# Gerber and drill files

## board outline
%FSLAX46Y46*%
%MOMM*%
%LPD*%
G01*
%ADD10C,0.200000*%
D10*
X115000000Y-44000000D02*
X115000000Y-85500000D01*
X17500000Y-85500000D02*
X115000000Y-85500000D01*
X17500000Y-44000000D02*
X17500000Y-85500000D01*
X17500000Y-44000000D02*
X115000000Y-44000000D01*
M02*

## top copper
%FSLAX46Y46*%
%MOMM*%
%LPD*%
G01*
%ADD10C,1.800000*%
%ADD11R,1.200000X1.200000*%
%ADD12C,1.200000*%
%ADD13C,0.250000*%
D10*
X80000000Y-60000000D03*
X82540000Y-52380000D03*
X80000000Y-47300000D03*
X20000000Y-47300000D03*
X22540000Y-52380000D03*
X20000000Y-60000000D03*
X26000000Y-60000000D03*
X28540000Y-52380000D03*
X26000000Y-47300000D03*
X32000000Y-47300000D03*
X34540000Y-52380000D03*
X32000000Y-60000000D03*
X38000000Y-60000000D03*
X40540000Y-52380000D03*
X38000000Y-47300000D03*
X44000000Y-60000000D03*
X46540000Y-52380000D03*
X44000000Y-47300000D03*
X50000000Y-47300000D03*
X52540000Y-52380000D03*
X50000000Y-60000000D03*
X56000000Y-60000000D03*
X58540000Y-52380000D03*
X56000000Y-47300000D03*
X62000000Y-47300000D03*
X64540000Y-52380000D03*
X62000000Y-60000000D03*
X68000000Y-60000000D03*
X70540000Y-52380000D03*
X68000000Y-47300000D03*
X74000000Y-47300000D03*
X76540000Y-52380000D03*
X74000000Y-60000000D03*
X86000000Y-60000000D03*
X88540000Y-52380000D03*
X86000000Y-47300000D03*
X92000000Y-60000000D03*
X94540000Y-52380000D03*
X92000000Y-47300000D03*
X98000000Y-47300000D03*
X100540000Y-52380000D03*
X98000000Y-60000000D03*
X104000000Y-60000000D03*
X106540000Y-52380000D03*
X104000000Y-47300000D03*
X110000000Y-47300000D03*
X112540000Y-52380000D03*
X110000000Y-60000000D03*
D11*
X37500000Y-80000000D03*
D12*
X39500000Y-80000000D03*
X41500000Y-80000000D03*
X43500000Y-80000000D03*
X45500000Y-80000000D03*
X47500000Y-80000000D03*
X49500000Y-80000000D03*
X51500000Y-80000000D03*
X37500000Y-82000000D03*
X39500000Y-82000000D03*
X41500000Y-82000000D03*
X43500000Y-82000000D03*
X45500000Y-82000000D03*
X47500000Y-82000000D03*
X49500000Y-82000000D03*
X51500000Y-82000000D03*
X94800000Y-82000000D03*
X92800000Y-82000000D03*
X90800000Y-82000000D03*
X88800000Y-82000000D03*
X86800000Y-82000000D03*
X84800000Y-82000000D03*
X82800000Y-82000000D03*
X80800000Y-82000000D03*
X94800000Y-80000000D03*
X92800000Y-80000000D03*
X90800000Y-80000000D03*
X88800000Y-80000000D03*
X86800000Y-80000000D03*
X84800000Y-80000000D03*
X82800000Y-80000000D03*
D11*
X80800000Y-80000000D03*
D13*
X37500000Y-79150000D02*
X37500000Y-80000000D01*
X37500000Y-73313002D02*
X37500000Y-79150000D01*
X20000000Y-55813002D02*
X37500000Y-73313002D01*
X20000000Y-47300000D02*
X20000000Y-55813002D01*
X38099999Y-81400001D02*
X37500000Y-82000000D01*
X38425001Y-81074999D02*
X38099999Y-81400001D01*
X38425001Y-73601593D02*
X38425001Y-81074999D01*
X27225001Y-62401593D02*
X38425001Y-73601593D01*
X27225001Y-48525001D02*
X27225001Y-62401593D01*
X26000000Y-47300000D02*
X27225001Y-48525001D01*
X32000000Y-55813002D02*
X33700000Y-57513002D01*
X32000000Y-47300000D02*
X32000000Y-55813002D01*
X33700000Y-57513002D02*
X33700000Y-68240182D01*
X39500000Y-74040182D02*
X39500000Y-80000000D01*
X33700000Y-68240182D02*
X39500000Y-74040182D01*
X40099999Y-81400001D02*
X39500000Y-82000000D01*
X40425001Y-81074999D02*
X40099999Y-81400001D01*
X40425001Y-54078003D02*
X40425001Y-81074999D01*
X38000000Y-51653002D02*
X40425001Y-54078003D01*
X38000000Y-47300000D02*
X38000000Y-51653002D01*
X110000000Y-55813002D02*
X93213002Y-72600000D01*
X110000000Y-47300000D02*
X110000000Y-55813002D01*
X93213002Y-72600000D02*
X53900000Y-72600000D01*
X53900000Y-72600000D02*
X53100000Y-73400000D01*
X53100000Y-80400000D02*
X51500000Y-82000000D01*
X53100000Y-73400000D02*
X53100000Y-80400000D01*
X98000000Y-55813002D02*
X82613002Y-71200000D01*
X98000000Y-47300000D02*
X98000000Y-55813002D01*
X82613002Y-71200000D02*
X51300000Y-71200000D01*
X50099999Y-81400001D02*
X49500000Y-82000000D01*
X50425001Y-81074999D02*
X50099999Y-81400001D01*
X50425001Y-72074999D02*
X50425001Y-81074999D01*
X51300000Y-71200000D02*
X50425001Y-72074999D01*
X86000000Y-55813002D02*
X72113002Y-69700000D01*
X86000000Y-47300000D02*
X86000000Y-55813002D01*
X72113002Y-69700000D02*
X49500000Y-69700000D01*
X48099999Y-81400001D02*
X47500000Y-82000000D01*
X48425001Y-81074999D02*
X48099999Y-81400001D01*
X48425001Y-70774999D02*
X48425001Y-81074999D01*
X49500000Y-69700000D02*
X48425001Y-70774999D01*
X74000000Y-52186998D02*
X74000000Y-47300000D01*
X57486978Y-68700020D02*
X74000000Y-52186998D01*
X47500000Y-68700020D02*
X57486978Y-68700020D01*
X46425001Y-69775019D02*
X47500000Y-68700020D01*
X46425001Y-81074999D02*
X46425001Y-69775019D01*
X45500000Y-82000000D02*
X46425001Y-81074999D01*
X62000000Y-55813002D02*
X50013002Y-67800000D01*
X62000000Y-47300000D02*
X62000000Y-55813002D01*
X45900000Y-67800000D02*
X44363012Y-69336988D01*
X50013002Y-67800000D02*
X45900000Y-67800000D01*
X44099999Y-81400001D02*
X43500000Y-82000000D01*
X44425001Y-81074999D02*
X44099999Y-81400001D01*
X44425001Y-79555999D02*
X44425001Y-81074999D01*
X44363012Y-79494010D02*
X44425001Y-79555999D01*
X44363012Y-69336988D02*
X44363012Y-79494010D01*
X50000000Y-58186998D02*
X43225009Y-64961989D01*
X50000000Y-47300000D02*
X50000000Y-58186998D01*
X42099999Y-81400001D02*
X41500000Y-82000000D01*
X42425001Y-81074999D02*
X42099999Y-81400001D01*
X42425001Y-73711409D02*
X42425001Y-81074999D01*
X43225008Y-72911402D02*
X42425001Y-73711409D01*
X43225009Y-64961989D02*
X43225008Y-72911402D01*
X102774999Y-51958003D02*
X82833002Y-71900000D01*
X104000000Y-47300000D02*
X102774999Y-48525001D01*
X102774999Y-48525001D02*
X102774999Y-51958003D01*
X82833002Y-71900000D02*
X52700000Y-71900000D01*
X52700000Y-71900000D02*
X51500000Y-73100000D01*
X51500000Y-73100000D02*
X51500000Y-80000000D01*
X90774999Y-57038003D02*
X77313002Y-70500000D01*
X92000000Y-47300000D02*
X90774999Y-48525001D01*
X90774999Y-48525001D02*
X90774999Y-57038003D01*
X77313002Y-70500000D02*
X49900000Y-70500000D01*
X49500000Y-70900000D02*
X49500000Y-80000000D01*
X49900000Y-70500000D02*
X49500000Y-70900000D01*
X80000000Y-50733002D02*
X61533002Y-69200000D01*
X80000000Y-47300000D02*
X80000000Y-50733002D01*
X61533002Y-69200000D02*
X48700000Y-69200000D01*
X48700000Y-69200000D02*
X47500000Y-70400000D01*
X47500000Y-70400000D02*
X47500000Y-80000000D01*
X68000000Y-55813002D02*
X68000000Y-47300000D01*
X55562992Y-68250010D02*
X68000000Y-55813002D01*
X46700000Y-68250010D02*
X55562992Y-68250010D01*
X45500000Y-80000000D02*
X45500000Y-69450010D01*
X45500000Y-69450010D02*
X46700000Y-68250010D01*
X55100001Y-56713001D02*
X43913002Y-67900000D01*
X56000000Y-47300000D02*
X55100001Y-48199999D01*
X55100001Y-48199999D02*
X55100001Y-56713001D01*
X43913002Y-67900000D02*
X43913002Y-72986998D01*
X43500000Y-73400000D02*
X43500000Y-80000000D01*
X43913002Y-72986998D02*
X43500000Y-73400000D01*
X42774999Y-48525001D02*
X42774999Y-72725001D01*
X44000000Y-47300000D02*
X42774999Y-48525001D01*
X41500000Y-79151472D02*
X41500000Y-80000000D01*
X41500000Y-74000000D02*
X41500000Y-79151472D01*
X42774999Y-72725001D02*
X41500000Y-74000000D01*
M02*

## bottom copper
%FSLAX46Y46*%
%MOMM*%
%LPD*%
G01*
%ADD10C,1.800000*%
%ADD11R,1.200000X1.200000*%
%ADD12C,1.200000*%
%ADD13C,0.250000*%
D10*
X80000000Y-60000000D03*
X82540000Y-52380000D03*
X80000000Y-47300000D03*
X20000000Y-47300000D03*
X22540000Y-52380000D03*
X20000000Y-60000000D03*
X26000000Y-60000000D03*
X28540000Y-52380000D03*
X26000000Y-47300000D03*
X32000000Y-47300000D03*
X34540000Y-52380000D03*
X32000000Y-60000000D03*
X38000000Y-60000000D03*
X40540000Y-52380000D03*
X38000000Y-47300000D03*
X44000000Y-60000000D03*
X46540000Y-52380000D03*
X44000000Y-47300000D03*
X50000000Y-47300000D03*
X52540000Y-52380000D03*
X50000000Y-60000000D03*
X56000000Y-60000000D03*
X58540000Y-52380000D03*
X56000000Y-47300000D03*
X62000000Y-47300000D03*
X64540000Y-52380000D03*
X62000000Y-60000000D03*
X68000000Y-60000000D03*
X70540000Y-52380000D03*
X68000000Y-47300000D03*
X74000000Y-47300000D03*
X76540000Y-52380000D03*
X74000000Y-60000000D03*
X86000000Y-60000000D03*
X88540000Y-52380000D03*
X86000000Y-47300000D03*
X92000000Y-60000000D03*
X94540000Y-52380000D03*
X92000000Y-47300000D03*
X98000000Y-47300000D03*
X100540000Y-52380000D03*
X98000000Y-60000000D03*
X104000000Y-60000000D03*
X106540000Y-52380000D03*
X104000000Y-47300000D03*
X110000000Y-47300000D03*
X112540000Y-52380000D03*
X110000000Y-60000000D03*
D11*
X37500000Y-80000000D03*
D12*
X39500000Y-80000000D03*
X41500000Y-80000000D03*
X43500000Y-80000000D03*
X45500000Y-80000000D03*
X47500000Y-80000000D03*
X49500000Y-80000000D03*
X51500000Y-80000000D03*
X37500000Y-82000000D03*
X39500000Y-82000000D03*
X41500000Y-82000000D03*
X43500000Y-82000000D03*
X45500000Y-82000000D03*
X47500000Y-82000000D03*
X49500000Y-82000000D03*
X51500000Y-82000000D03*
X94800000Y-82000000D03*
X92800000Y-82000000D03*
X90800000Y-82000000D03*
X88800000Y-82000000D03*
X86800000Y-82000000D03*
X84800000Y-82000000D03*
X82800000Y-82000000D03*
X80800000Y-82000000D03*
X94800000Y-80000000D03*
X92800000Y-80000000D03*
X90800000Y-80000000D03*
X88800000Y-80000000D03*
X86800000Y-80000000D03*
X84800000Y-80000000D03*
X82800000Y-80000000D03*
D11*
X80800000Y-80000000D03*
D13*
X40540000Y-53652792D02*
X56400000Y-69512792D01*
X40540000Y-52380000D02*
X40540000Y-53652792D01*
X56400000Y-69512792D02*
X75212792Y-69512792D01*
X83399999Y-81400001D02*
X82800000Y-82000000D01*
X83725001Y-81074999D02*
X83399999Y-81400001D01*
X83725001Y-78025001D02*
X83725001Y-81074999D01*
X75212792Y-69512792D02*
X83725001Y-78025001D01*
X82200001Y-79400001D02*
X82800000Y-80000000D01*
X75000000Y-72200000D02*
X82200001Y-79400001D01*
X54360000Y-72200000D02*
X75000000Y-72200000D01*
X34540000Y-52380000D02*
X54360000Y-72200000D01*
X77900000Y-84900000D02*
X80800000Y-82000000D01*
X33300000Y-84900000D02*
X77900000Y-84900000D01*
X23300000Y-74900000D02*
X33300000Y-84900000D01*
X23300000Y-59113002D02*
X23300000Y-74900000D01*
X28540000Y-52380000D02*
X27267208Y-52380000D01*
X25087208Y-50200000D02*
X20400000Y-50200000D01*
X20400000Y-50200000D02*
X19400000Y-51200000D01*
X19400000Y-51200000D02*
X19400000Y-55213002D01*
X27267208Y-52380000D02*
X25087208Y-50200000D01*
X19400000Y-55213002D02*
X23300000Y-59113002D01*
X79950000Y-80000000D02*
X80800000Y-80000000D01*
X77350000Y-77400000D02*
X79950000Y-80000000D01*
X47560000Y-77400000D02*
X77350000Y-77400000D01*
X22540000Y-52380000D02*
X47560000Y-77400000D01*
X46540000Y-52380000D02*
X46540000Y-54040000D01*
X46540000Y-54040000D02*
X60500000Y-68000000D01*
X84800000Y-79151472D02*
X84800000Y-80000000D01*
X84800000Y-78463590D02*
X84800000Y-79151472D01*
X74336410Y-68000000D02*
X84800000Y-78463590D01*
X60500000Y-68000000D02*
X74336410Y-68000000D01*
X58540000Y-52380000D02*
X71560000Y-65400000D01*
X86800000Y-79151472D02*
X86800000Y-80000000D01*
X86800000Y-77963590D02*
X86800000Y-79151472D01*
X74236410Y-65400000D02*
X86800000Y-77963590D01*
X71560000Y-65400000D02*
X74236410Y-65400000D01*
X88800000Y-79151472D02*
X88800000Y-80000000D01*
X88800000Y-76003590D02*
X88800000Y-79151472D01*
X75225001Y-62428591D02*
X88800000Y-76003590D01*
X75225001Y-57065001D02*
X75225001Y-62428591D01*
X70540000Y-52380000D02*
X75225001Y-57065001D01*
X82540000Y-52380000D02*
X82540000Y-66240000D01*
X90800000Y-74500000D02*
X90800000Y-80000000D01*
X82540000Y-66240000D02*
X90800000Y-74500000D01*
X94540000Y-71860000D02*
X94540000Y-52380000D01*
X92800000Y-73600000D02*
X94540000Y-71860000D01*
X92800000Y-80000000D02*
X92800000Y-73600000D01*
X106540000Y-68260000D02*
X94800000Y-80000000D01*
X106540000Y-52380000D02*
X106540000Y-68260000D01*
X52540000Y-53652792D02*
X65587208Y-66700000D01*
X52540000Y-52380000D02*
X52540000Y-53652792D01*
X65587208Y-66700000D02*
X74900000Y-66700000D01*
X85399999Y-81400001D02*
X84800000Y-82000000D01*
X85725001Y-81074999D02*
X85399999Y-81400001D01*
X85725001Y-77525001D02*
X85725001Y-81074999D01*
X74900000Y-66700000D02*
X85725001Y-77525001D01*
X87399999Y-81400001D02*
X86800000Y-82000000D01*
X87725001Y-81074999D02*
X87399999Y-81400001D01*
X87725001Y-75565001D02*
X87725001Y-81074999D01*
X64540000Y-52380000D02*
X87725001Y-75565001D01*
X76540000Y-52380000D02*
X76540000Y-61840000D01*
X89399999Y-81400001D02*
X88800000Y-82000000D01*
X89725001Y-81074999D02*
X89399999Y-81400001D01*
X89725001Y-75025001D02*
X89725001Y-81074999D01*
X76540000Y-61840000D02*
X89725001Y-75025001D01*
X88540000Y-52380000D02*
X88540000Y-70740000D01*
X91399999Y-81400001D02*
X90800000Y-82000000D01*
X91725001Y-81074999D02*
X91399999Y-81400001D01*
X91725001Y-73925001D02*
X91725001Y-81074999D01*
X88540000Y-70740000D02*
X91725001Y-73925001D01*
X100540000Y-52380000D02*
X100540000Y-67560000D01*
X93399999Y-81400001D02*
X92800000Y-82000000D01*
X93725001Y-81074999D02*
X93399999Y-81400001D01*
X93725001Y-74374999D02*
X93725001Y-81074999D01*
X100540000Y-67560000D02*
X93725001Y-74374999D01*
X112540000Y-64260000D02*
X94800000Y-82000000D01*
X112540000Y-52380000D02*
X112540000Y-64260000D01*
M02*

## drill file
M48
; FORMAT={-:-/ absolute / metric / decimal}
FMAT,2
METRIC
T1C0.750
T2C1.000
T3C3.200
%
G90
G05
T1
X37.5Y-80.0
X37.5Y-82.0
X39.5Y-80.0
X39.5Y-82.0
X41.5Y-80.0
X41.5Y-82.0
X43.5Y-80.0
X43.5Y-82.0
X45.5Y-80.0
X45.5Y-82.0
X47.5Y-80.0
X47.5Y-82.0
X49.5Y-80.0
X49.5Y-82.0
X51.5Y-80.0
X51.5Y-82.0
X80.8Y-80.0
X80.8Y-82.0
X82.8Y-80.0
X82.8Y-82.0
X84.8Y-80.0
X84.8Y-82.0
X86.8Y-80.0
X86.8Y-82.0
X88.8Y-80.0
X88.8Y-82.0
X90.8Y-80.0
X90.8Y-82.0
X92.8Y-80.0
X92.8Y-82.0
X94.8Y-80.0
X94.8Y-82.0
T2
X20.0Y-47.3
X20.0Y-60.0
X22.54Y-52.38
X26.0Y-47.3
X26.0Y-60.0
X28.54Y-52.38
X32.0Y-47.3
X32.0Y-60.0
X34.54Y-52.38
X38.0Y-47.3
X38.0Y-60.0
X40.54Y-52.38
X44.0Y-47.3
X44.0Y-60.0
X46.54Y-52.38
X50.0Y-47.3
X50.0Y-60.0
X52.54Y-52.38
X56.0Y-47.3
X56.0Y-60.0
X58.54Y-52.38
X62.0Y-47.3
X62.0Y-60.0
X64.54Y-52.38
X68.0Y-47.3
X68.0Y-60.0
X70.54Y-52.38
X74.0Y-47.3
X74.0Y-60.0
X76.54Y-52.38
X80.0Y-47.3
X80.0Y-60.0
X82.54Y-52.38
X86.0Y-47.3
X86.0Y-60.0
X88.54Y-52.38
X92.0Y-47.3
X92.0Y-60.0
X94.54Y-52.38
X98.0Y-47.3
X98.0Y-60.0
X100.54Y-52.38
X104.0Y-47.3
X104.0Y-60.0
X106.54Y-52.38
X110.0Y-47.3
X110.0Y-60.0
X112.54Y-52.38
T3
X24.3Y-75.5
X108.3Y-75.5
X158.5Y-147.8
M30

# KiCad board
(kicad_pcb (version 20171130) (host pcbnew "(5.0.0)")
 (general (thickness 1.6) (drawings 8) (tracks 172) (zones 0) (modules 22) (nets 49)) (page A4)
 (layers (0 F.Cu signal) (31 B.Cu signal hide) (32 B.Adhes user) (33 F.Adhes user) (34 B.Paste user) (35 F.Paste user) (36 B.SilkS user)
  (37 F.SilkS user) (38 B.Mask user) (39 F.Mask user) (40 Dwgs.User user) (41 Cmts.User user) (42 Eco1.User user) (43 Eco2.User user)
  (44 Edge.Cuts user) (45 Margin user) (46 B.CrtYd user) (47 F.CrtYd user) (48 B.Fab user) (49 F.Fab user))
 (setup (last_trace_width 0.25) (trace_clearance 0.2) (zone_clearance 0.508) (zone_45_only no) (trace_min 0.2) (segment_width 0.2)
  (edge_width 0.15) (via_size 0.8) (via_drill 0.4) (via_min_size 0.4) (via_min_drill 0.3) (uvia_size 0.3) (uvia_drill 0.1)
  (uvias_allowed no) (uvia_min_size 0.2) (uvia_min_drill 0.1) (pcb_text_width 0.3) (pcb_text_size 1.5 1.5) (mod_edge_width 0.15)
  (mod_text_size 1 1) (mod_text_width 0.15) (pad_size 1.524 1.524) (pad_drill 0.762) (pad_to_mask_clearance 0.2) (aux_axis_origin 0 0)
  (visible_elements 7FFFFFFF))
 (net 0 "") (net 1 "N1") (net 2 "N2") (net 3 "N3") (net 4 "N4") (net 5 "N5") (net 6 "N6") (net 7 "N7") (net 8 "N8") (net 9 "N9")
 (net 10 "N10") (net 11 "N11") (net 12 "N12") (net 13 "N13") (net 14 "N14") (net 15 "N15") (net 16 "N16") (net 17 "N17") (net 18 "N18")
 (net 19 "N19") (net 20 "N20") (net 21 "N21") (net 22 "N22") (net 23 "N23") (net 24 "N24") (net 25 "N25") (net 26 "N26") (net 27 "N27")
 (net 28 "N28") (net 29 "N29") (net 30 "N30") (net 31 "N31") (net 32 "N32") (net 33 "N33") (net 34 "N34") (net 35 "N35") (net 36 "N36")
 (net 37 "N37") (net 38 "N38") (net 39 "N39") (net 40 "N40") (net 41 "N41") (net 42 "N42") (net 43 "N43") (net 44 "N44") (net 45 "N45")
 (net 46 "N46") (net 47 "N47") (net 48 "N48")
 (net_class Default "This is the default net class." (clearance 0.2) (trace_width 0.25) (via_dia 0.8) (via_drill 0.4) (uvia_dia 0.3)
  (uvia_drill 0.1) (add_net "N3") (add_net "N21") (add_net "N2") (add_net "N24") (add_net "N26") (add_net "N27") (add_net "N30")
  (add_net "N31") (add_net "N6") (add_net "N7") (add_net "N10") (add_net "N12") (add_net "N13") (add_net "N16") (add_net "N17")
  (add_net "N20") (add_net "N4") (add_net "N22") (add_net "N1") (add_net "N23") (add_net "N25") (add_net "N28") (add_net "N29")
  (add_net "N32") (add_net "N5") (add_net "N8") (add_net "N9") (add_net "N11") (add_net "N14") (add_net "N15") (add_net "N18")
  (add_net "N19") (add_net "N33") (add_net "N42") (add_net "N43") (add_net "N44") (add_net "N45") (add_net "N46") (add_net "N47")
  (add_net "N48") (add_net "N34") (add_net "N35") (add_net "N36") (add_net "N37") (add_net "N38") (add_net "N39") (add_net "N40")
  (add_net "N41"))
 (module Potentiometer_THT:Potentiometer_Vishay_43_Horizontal (layer F.Cu) (at 80 60 270)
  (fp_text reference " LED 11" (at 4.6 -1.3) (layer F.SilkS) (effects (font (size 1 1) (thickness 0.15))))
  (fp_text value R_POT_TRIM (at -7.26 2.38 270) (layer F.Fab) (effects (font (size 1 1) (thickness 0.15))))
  (pad 1 thru_hole circle (at 0 0 270) (size 1.8 1.8) (drill 1) (layers *.Cu *.Mask))
  (pad 2 thru_hole circle (at -7.62 -2.54 270) (size 1.8 1.8) (drill 1) (layers *.Cu *.Mask) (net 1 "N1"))
  (pad 3 thru_hole circle (at -12.7 0 270) (size 1.8 1.8) (drill 1) (layers *.Cu *.Mask) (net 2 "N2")))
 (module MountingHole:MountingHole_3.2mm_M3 (layer F.Cu) (at 108.3 75.5)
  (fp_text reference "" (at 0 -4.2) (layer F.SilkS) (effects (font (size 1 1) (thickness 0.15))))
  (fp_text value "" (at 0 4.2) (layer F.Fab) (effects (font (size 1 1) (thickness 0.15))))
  (pad 1 np_thru_hole circle (at 0 0) (size 3.2 3.2) (drill 3.2) (layers *.Cu *.Mask)))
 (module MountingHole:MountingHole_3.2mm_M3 (layer F.Cu) (at 24.3 75.5)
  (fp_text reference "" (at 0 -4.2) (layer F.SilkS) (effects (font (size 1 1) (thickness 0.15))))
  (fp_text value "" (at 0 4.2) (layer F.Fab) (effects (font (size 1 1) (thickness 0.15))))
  (pad 1 np_thru_hole circle (at 0 0) (size 3.2 3.2) (drill 3.2) (layers *.Cu *.Mask)))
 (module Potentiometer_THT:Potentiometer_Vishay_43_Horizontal (layer F.Cu) (at 20 60 270)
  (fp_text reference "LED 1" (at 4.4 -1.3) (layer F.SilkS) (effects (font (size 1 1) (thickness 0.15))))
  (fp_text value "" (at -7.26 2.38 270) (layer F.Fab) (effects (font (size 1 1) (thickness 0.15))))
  (pad 3 thru_hole circle (at -12.7 0 270) (size 1.8 1.8) (drill 1) (layers *.Cu *.Mask) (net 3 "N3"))
  (pad 2 thru_hole circle (at -7.62 -2.54 270) (size 1.8 1.8) (drill 1) (layers *.Cu *.Mask) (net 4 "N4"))
  (pad 1 thru_hole circle (at 0 0 270) (size 1.8 1.8) (drill 1) (layers *.Cu *.Mask)))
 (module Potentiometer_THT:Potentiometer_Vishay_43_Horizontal (layer F.Cu) (at 26 60 270)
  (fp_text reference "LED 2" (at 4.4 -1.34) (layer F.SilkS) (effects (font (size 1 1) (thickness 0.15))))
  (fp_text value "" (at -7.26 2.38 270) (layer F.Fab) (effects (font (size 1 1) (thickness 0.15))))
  (pad 1 thru_hole circle (at 0 0 270) (size 1.8 1.8) (drill 1) (layers *.Cu *.Mask))
  (pad 2 thru_hole circle (at -7.62 -2.54 270) (size 1.8 1.8) (drill 1) (layers *.Cu *.Mask) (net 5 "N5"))
  (pad 3 thru_hole circle (at -12.7 0 270) (size 1.8 1.8) (drill 1) (layers *.Cu *.Mask) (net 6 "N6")))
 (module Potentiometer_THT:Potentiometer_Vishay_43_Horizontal (layer F.Cu) (at 32 60 270)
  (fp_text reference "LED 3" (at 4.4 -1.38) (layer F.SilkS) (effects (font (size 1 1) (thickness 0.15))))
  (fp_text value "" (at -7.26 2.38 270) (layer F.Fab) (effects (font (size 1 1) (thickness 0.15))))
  (pad 3 thru_hole circle (at -12.7 0 270) (size 1.8 1.8) (drill 1) (layers *.Cu *.Mask) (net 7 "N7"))
  (pad 2 thru_hole circle (at -7.62 -2.54 270) (size 1.8 1.8) (drill 1) (layers *.Cu *.Mask) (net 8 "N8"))
  (pad 1 thru_hole circle (at 0 0 270) (size 1.8 1.8) (drill 1) (layers *.Cu *.Mask)))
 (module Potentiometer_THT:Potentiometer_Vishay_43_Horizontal (layer F.Cu) (at 38 60 270)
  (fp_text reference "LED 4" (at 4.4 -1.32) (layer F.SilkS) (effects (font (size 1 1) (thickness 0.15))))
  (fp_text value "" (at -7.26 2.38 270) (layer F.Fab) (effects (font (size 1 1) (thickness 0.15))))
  (pad 1 thru_hole circle (at 0 0 270) (size 1.8 1.8) (drill 1) (layers *.Cu *.Mask))
  (pad 2 thru_hole circle (at -7.62 -2.54 270) (size 1.8 1.8) (drill 1) (layers *.Cu *.Mask) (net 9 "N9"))
  (pad 3 thru_hole circle (at -12.7 0 270) (size 1.8 1.8) (drill 1) (layers *.Cu *.Mask) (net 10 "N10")))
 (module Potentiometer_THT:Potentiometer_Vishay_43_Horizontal (layer F.Cu) (at 44 60 270)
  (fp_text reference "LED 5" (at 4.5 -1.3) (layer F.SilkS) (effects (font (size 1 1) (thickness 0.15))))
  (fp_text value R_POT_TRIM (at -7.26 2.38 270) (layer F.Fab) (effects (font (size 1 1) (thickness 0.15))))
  (pad 1 thru_hole circle (at 0 0 270) (size 1.8 1.8) (drill 1) (layers *.Cu *.Mask))
  (pad 2 thru_hole circle (at -7.62 -2.54 270) (size 1.8 1.8) (drill 1) (layers *.Cu *.Mask) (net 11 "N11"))
  (pad 3 thru_hole circle (at -12.7 0 270) (size 1.8 1.8) (drill 1) (layers *.Cu *.Mask) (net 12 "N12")))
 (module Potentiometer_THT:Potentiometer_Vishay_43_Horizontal (layer F.Cu) (at 50 60 270)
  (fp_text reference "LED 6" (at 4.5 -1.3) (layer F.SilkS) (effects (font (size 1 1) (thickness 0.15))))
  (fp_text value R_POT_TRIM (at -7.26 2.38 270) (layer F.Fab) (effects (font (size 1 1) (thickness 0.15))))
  (pad 3 thru_hole circle (at -12.7 0 270) (size 1.8 1.8) (drill 1) (layers *.Cu *.Mask) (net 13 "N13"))
  (pad 2 thru_hole circle (at -7.62 -2.54 270) (size 1.8 1.8) (drill 1) (layers *.Cu *.Mask) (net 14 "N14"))
  (pad 1 thru_hole circle (at 0 0 270) (size 1.8 1.8) (drill 1) (layers *.Cu *.Mask)))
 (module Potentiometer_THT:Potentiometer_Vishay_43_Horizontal (layer F.Cu) (at 56 60 270)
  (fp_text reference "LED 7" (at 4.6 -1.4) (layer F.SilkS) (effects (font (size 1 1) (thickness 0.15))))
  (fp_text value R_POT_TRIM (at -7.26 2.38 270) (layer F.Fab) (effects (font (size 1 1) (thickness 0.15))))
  (pad 1 thru_hole circle (at 0 0 270) (size 1.8 1.8) (drill 1) (layers *.Cu *.Mask))
  (pad 2 thru_hole circle (at -7.62 -2.54 270) (size 1.8 1.8) (drill 1) (layers *.Cu *.Mask) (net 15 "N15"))
  (pad 3 thru_hole circle (at -12.7 0 270) (size 1.8 1.8) (drill 1) (layers *.Cu *.Mask) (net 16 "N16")))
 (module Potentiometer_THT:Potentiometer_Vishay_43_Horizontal (layer F.Cu) (at 62 60 270)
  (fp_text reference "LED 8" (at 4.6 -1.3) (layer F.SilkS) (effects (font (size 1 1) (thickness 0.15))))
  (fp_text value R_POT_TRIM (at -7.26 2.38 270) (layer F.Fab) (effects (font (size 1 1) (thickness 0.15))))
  (pad 3 thru_hole circle (at -12.7 0 270) (size 1.8 1.8) (drill 1) (layers *.Cu *.Mask) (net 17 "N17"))
  (pad 2 thru_hole circle (at -7.62 -2.54 270) (size 1.8 1.8) (drill 1) (layers *.Cu *.Mask) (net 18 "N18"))
  (pad 1 thru_hole circle (at 0 0 270) (size 1.8 1.8) (drill 1) (layers *.Cu *.Mask)))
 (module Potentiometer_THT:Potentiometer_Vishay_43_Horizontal (layer F.Cu) (at 68 60 270)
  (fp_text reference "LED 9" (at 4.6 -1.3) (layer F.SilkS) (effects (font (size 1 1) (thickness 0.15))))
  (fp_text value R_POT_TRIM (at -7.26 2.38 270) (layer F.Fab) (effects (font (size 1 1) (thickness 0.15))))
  (pad 1 thru_hole circle (at 0 0 270) (size 1.8 1.8) (drill 1) (layers *.Cu *.Mask))
  (pad 2 thru_hole circle (at -7.62 -2.54 270) (size 1.8 1.8) (drill 1) (layers *.Cu *.Mask) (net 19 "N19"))
  (pad 3 thru_hole circle (at -12.7 0 270) (size 1.8 1.8) (drill 1) (layers *.Cu *.Mask) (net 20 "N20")))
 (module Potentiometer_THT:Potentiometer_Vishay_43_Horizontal (layer F.Cu) (at 74 60 270)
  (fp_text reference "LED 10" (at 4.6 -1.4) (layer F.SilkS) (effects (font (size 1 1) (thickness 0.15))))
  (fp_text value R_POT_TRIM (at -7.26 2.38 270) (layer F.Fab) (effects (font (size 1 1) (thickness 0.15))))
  (pad 3 thru_hole circle (at -12.7 0 270) (size 1.8 1.8) (drill 1) (layers *.Cu *.Mask) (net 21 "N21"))
  (pad 2 thru_hole circle (at -7.62 -2.54 270) (size 1.8 1.8) (drill 1) (layers *.Cu *.Mask) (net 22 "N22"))
  (pad 1 thru_hole circle (at 0 0 270) (size 1.8 1.8) (drill 1) (layers *.Cu *.Mask)))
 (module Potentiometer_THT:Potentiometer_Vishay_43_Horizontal (layer F.Cu) (at 86 60 270)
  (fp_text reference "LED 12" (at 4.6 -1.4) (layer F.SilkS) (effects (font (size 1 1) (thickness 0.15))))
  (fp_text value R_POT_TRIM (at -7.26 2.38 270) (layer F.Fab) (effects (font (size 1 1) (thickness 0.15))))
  (pad 1 thru_hole circle (at 0 0 270) (size 1.8 1.8) (drill 1) (layers *.Cu *.Mask))
  (pad 2 thru_hole circle (at -7.62 -2.54 270) (size 1.8 1.8) (drill 1) (layers *.Cu *.Mask) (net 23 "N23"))
  (pad 3 thru_hole circle (at -12.7 0 270) (size 1.8 1.8) (drill 1) (layers *.Cu *.Mask) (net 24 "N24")))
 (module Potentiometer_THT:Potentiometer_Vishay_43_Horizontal (layer F.Cu) (at 92 60 270)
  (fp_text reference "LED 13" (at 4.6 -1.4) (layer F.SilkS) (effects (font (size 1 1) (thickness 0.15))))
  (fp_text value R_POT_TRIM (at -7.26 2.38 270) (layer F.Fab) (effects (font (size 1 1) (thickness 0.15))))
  (pad 1 thru_hole circle (at 0 0 270) (size 1.8 1.8) (drill 1) (layers *.Cu *.Mask))
  (pad 2 thru_hole circle (at -7.62 -2.54 270) (size 1.8 1.8) (drill 1) (layers *.Cu *.Mask) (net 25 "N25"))
  (pad 3 thru_hole circle (at -12.7 0 270) (size 1.8 1.8) (drill 1) (layers *.Cu *.Mask) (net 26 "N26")))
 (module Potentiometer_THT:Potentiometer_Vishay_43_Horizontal (layer F.Cu) (at 98 60 270)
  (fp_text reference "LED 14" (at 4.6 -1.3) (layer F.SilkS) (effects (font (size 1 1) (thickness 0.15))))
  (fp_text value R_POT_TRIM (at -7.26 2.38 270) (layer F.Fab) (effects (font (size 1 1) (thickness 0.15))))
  (pad 3 thru_hole circle (at -12.7 0 270) (size 1.8 1.8) (drill 1) (layers *.Cu *.Mask) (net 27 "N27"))
  (pad 2 thru_hole circle (at -7.62 -2.54 270) (size 1.8 1.8) (drill 1) (layers *.Cu *.Mask) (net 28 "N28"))
  (pad 1 thru_hole circle (at 0 0 270) (size 1.8 1.8) (drill 1) (layers *.Cu *.Mask)))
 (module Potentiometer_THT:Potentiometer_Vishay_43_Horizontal (layer F.Cu) (at 104 60 270)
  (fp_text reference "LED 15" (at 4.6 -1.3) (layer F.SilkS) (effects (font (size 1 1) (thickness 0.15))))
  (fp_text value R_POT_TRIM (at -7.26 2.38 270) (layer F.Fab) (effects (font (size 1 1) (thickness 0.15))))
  (pad 1 thru_hole circle (at 0 0 270) (size 1.8 1.8) (drill 1) (layers *.Cu *.Mask))
  (pad 2 thru_hole circle (at -7.62 -2.54 270) (size 1.8 1.8) (drill 1) (layers *.Cu *.Mask) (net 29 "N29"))
  (pad 3 thru_hole circle (at -12.7 0 270) (size 1.8 1.8) (drill 1) (layers *.Cu *.Mask) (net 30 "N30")))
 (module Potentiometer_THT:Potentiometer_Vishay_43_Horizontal (layer F.Cu) (at 110 60 270)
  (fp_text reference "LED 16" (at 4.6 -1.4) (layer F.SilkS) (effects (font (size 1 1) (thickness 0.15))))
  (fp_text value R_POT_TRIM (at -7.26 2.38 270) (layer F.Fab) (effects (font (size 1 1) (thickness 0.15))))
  (pad 3 thru_hole circle (at -12.7 0 270) (size 1.8 1.8) (drill 1) (layers *.Cu *.Mask) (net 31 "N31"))
  (pad 2 thru_hole circle (at -7.62 -2.54 270) (size 1.8 1.8) (drill 1) (layers *.Cu *.Mask) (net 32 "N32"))
  (pad 1 thru_hole circle (at 0 0 270) (size 1.8 1.8) (drill 1) (layers *.Cu *.Mask)))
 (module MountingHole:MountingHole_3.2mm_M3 (layer F.Cu) (at 158.5 147.8)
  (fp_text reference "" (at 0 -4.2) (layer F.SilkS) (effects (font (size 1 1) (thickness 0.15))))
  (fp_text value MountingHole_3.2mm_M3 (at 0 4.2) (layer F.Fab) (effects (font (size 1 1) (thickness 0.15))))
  (pad 1 np_thru_hole circle (at 0 0) (size 3.2 3.2) (drill 3.2) (layers *.Cu *.Mask)))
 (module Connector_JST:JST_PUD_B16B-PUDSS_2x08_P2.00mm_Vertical (layer F.Cu) (at 37.5 80)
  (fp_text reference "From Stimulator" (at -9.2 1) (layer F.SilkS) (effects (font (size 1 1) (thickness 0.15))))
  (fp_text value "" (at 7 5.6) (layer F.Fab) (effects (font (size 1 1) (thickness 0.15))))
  (pad 1 thru_hole rect (at 0 0) (size 1.2 1.2) (drill 0.75) (layers *.Cu *.Mask) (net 3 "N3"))
  (pad 3 thru_hole circle (at 2 0) (size 1.2 1.2) (drill 0.75) (layers *.Cu *.Mask) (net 7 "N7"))
  (pad 5 thru_hole circle (at 4 0) (size 1.2 1.2) (drill 0.75) (layers *.Cu *.Mask) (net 12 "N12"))
  (pad 7 thru_hole circle (at 6 0) (size 1.2 1.2) (drill 0.75) (layers *.Cu *.Mask) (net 16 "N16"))
  (pad 9 thru_hole circle (at 8 0) (size 1.2 1.2) (drill 0.75) (layers *.Cu *.Mask) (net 20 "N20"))
  (pad 11 thru_hole circle (at 10 0) (size 1.2 1.2) (drill 0.75) (layers *.Cu *.Mask) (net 2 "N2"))
  (pad 13 thru_hole circle (at 12 0) (size 1.2 1.2) (drill 0.75) (layers *.Cu *.Mask) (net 26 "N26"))
  (pad 15 thru_hole circle (at 14 0) (size 1.2 1.2) (drill 0.75) (layers *.Cu *.Mask) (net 30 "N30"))
  (pad 2 thru_hole circle (at 0 2) (size 1.2 1.2) (drill 0.75) (layers *.Cu *.Mask) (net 6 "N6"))
  (pad 4 thru_hole circle (at 2 2) (size 1.2 1.2) (drill 0.75) (layers *.Cu *.Mask) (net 10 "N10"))
  (pad 6 thru_hole circle (at 4 2) (size 1.2 1.2) (drill 0.75) (layers *.Cu *.Mask) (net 13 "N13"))
  (pad 8 thru_hole circle (at 6 2) (size 1.2 1.2) (drill 0.75) (layers *.Cu *.Mask) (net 17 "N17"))
  (pad 10 thru_hole circle (at 8 2) (size 1.2 1.2) (drill 0.75) (layers *.Cu *.Mask) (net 21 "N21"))
  (pad 12 thru_hole circle (at 10 2) (size 1.2 1.2) (drill 0.75) (layers *.Cu *.Mask) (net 24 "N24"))
  (pad 14 thru_hole circle (at 12 2) (size 1.2 1.2) (drill 0.75) (layers *.Cu *.Mask) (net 27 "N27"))
  (pad 16 thru_hole circle (at 14 2) (size 1.2 1.2) (drill 0.75) (layers *.Cu *.Mask) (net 31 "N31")))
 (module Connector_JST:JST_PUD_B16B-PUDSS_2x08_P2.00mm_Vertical (layer F.Cu) (at 80.8 80)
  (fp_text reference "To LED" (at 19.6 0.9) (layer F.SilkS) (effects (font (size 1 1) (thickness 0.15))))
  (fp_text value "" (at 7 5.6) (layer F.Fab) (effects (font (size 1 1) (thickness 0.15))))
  (pad 16 thru_hole circle (at 14 2) (size 1.2 1.2) (drill 0.75) (layers *.Cu *.Mask) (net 32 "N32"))
  (pad 14 thru_hole circle (at 12 2) (size 1.2 1.2) (drill 0.75) (layers *.Cu *.Mask) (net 28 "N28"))
  (pad 12 thru_hole circle (at 10 2) (size 1.2 1.2) (drill 0.75) (layers *.Cu *.Mask) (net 23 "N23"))
  (pad 10 thru_hole circle (at 8 2) (size 1.2 1.2) (drill 0.75) (layers *.Cu *.Mask) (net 22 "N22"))
  (pad 8 thru_hole circle (at 6 2) (size 1.2 1.2) (drill 0.75) (layers *.Cu *.Mask) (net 18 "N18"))
  (pad 6 thru_hole circle (at 4 2) (size 1.2 1.2) (drill 0.75) (layers *.Cu *.Mask) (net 14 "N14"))
  (pad 4 thru_hole circle (at 2 2) (size 1.2 1.2) (drill 0.75) (layers *.Cu *.Mask) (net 9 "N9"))
  (pad 2 thru_hole circle (at 0 2) (size 1.2 1.2) (drill 0.75) (layers *.Cu *.Mask) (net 5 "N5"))
  (pad 15 thru_hole circle (at 14 0) (size 1.2 1.2) (drill 0.75) (layers *.Cu *.Mask) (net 29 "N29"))
  (pad 13 thru_hole circle (at 12 0) (size 1.2 1.2) (drill 0.75) (layers *.Cu *.Mask) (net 25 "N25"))
  (pad 11 thru_hole circle (at 10 0) (size 1.2 1.2) (drill 0.75) (layers *.Cu *.Mask) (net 1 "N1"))
  (pad 9 thru_hole circle (at 8 0) (size 1.2 1.2) (drill 0.75) (layers *.Cu *.Mask) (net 19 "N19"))
  (pad 7 thru_hole circle (at 6 0) (size 1.2 1.2) (drill 0.75) (layers *.Cu *.Mask) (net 15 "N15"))
  (pad 5 thru_hole circle (at 4 0) (size 1.2 1.2) (drill 0.75) (layers *.Cu *.Mask) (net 11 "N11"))
  (pad 3 thru_hole circle (at 2 0) (size 1.2 1.2) (drill 0.75) (layers *.Cu *.Mask) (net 8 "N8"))
  (pad 1 thru_hole rect (at 0 0) (size 1.2 1.2) (drill 0.75) (layers *.Cu *.Mask) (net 4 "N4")))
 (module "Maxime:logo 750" (layer F.Cu) (at 67.8 80.4)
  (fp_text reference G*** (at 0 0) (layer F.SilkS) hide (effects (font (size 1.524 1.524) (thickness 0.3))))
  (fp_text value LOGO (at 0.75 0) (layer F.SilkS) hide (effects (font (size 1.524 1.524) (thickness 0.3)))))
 (gr_line (start 115 44) (end 115 85.5) (layer Edge.Cuts) (width 0.2))
 (gr_line (start 17.5 85.5) (end 115 85.5) (layer Edge.Cuts) (width 0.2))
 (gr_line (start 17.5 44) (end 17.5 85.5) (layer Edge.Cuts) (width 0.2))
 (gr_line (start 17.5 44) (end 115 44) (layer Edge.Cuts) (width 0.2))
 (segment (start 37.5 79.15) (end 37.5 80) (width 0.25) (layer F.Cu) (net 3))
 (segment (start 37.5 73.313002) (end 37.5 79.15) (width 0.25) (layer F.Cu) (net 3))
 (segment (start 20 55.813002) (end 37.5 73.313002) (width 0.25) (layer F.Cu) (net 3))
 (segment (start 20 47.3) (end 20 55.813002) (width 0.25) (layer F.Cu) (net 3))
 (segment (start 38.099999 81.400001) (end 37.5 82) (width 0.25) (layer F.Cu) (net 6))
 (segment (start 38.425001 81.074999) (end 38.099999 81.400001) (width 0.25) (layer F.Cu) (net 6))
 (segment (start 38.425001 73.601593) (end 38.425001 81.074999) (width 0.25) (layer F.Cu) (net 6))
 (segment (start 27.225001 62.401593) (end 38.425001 73.601593) (width 0.25) (layer F.Cu) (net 6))
 (segment (start 27.225001 48.525001) (end 27.225001 62.401593) (width 0.25) (layer F.Cu) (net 6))
 (segment (start 26 47.3) (end 27.225001 48.525001) (width 0.25) (layer F.Cu) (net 6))
 (segment (start 32 55.813002) (end 33.7 57.513002) (width 0.25) (layer F.Cu) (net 7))
 (segment (start 32 47.3) (end 32 55.813002) (width 0.25) (layer F.Cu) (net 7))
 (segment (start 33.7 57.513002) (end 33.7 68.240182) (width 0.25) (layer F.Cu) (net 7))
 (segment (start 39.5 74.040182) (end 39.5 80) (width 0.25) (layer F.Cu) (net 7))
 (segment (start 33.7 68.240182) (end 39.5 74.040182) (width 0.25) (layer F.Cu) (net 7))
 (segment (start 40.099999 81.400001) (end 39.5 82) (width 0.25) (layer F.Cu) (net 10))
 (segment (start 40.425001 81.074999) (end 40.099999 81.400001) (width 0.25) (layer F.Cu) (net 10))
 (segment (start 40.425001 54.078003) (end 40.425001 81.074999) (width 0.25) (layer F.Cu) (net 10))
 (segment (start 38 51.653002) (end 40.425001 54.078003) (width 0.25) (layer F.Cu) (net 10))
 (segment (start 38 47.3) (end 38 51.653002) (width 0.25) (layer F.Cu) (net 10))
 (segment (start 40.54 53.652792) (end 56.4 69.512792) (width 0.25) (layer B.Cu) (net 9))
 (segment (start 40.54 52.38) (end 40.54 53.652792) (width 0.25) (layer B.Cu) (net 9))
 (segment (start 56.4 69.512792) (end 75.212792 69.512792) (width 0.25) (layer B.Cu) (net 9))
 (segment (start 83.399999 81.400001) (end 82.8 82) (width 0.25) (layer B.Cu) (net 9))
 (segment (start 83.725001 81.074999) (end 83.399999 81.400001) (width 0.25) (layer B.Cu) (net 9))
 (segment (start 83.725001 78.025001) (end 83.725001 81.074999) (width 0.25) (layer B.Cu) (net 9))
 (segment (start 75.212792 69.512792) (end 83.725001 78.025001) (width 0.25) (layer B.Cu) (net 9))
 (segment (start 82.200001 79.400001) (end 82.8 80) (width 0.25) (layer B.Cu) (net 8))
 (segment (start 75 72.2) (end 82.200001 79.400001) (width 0.25) (layer B.Cu) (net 8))
 (segment (start 54.36 72.2) (end 75 72.2) (width 0.25) (layer B.Cu) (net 8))
 (segment (start 34.54 52.38) (end 54.36 72.2) (width 0.25) (layer B.Cu) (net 8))
 (segment (start 77.9 84.9) (end 80.8 82) (width 0.25) (layer B.Cu) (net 5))
 (segment (start 33.3 84.9) (end 77.9 84.9) (width 0.25) (layer B.Cu) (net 5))
 (segment (start 23.3 74.9) (end 33.3 84.9) (width 0.25) (layer B.Cu) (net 5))
 (segment (start 23.3 59.113002) (end 23.3 74.9) (width 0.25) (layer B.Cu) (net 5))
 (segment (start 28.54 52.38) (end 27.267208 52.38) (width 0.25) (layer B.Cu) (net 5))
 (segment (start 25.087208 50.2) (end 20.4 50.2) (width 0.25) (layer B.Cu) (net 5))
 (segment (start 20.4 50.2) (end 19.4 51.2) (width 0.25) (layer B.Cu) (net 5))
 (segment (start 19.4 51.2) (end 19.4 55.213002) (width 0.25) (layer B.Cu) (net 5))
 (segment (start 27.267208 52.38) (end 25.087208 50.2) (width 0.25) (layer B.Cu) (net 5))
 (segment (start 19.4 55.213002) (end 23.3 59.113002) (width 0.25) (layer B.Cu) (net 5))
 (segment (start 79.95 80) (end 80.8 80) (width 0.25) (layer B.Cu) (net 4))
 (segment (start 77.35 77.4) (end 79.95 80) (width 0.25) (layer B.Cu) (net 4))
 (segment (start 47.56 77.4) (end 77.35 77.4) (width 0.25) (layer B.Cu) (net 4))
 (segment (start 22.54 52.38) (end 47.56 77.4) (width 0.25) (layer B.Cu) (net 4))
 (segment (start 110 55.813002) (end 93.213002 72.6) (width 0.25) (layer F.Cu) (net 31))
 (segment (start 110 47.3) (end 110 55.813002) (width 0.25) (layer F.Cu) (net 31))
 (segment (start 93.213002 72.6) (end 53.9 72.6) (width 0.25) (layer F.Cu) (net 31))
 (segment (start 53.9 72.6) (end 53.1 73.4) (width 0.25) (layer F.Cu) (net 31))
 (segment (start 53.1 80.4) (end 51.5 82) (width 0.25) (layer F.Cu) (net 31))
 (segment (start 53.1 73.4) (end 53.1 80.4) (width 0.25) (layer F.Cu) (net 31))
 (segment (start 98 55.813002) (end 82.613002 71.2) (width 0.25) (layer F.Cu) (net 27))
 (segment (start 98 47.3) (end 98 55.813002) (width 0.25) (layer F.Cu) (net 27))
 (segment (start 82.613002 71.2) (end 51.3 71.2) (width 0.25) (layer F.Cu) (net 27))
 (segment (start 50.099999 81.400001) (end 49.5 82) (width 0.25) (layer F.Cu) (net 27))
 (segment (start 50.425001 81.074999) (end 50.099999 81.400001) (width 0.25) (layer F.Cu) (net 27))
 (segment (start 50.425001 72.074999) (end 50.425001 81.074999) (width 0.25) (layer F.Cu) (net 27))
 (segment (start 51.3 71.2) (end 50.425001 72.074999) (width 0.25) (layer F.Cu) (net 27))
 (segment (start 86 55.813002) (end 72.113002 69.7) (width 0.25) (layer F.Cu) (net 24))
 (segment (start 86 47.3) (end 86 55.813002) (width 0.25) (layer F.Cu) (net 24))
 (segment (start 72.113002 69.7) (end 49.5 69.7) (width 0.25) (layer F.Cu) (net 24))
 (segment (start 48.099999 81.400001) (end 47.5 82) (width 0.25) (layer F.Cu) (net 24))
 (segment (start 48.425001 81.074999) (end 48.099999 81.400001) (width 0.25) (layer F.Cu) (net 24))
 (segment (start 48.425001 70.774999) (end 48.425001 81.074999) (width 0.25) (layer F.Cu) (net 24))
 (segment (start 49.5 69.7) (end 48.425001 70.774999) (width 0.25) (layer F.Cu) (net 24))
 (segment (start 74 52.186998) (end 74 47.3) (width 0.25) (layer F.Cu) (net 21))
 (segment (start 57.486978 68.70002) (end 74 52.186998) (width 0.25) (layer F.Cu) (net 21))
 (segment (start 47.5 68.70002) (end 57.486978 68.70002) (width 0.25) (layer F.Cu) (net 21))
 (segment (start 46.425001 69.775019) (end 47.5 68.70002) (width 0.25) (layer F.Cu) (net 21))
 (segment (start 46.425001 81.074999) (end 46.425001 69.775019) (width 0.25) (layer F.Cu) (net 21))
 (segment (start 45.5 82) (end 46.425001 81.074999) (width 0.25) (layer F.Cu) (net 21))
 (segment (start 62 55.813002) (end 50.013002 67.8) (width 0.25) (layer F.Cu) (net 17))
 (segment (start 62 47.3) (end 62 55.813002) (width 0.25) (layer F.Cu) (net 17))
 (segment (start 45.9 67.8) (end 44.363012 69.336988) (width 0.25) (layer F.Cu) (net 17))
 (segment (start 50.013002 67.8) (end 45.9 67.8) (width 0.25) (layer F.Cu) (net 17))
 (segment (start 44.099999 81.400001) (end 43.5 82) (width 0.25) (layer F.Cu) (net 17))
 (segment (start 44.425001 81.074999) (end 44.099999 81.400001) (width 0.25) (layer F.Cu) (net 17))
 (segment (start 44.425001 79.555999) (end 44.425001 81.074999) (width 0.25) (layer F.Cu) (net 17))
 (segment (start 44.363012 79.49401) (end 44.425001 79.555999) (width 0.25) (layer F.Cu) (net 17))
 (segment (start 44.363012 69.336988) (end 44.363012 79.49401) (width 0.25) (layer F.Cu) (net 17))
 (segment (start 50 58.186998) (end 43.225009 64.961989) (width 0.25) (layer F.Cu) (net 13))
 (segment (start 50 47.3) (end 50 58.186998) (width 0.25) (layer F.Cu) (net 13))
 (segment (start 42.099999 81.400001) (end 41.5 82) (width 0.25) (layer F.Cu) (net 13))
 (segment (start 42.425001 81.074999) (end 42.099999 81.400001) (width 0.25) (layer F.Cu) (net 13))
 (segment (start 42.425001 73.711409) (end 42.425001 81.074999) (width 0.25) (layer F.Cu) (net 13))
 (segment (start 43.225008 72.911402) (end 42.425001 73.711409) (width 0.25) (layer F.Cu) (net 13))
 (segment (start 43.225009 64.961989) (end 43.225008 72.911402) (width 0.25) (layer F.Cu) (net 13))
 (segment (start 102.774999 51.958003) (end 82.833002 71.9) (width 0.25) (layer F.Cu) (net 30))
 (segment (start 104 47.3) (end 102.774999 48.525001) (width 0.25) (layer F.Cu) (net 30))
 (segment (start 102.774999 48.525001) (end 102.774999 51.958003) (width 0.25) (layer F.Cu) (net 30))
 (segment (start 82.833002 71.9) (end 52.7 71.9) (width 0.25) (layer F.Cu) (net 30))
 (segment (start 52.7 71.9) (end 51.5 73.1) (width 0.25) (layer F.Cu) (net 30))
 (segment (start 51.5 73.1) (end 51.5 80) (width 0.25) (layer F.Cu) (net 30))
 (segment (start 90.774999 57.038003) (end 77.313002 70.5) (width 0.25) (layer F.Cu) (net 26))
 (segment (start 92 47.3) (end 90.774999 48.525001) (width 0.25) (layer F.Cu) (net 26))
 (segment (start 90.774999 48.525001) (end 90.774999 57.038003) (width 0.25) (layer F.Cu) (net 26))
 (segment (start 77.313002 70.5) (end 49.9 70.5) (width 0.25) (layer F.Cu) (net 26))
 (segment (start 49.5 70.9) (end 49.5 80) (width 0.25) (layer F.Cu) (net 26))
 (segment (start 49.9 70.5) (end 49.5 70.9) (width 0.25) (layer F.Cu) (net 26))
 (segment (start 80 50.733002) (end 61.533002 69.2) (width 0.25) (layer F.Cu) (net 2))
 (segment (start 80 47.3) (end 80 50.733002) (width 0.25) (layer F.Cu) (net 2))
 (segment (start 61.533002 69.2) (end 48.7 69.2) (width 0.25) (layer F.Cu) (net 2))
 (segment (start 48.7 69.2) (end 47.5 70.4) (width 0.25) (layer F.Cu) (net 2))
 (segment (start 47.5 70.4) (end 47.5 80) (width 0.25) (layer F.Cu) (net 2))
 (segment (start 68 55.813002) (end 68 47.3) (width 0.25) (layer F.Cu) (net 20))
 (segment (start 55.562992 68.25001) (end 68 55.813002) (width 0.25) (layer F.Cu) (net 20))
 (segment (start 46.7 68.25001) (end 55.562992 68.25001) (width 0.25) (layer F.Cu) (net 20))
 (segment (start 45.5 80) (end 45.5 69.45001) (width 0.25) (layer F.Cu) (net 20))
 (segment (start 45.5 69.45001) (end 46.7 68.25001) (width 0.25) (layer F.Cu) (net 20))
 (segment (start 55.100001 56.713001) (end 43.913002 67.9) (width 0.25) (layer F.Cu) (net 16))
 (segment (start 56 47.3) (end 55.100001 48.199999) (width 0.25) (layer F.Cu) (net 16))
 (segment (start 55.100001 48.199999) (end 55.100001 56.713001) (width 0.25) (layer F.Cu) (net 16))
 (segment (start 43.913002 67.9) (end 43.913002 72.986998) (width 0.25) (layer F.Cu) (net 16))
 (segment (start 43.5 73.4) (end 43.5 80) (width 0.25) (layer F.Cu) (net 16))
 (segment (start 43.913002 72.986998) (end 43.5 73.4) (width 0.25) (layer F.Cu) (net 16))
 (segment (start 42.774999 48.525001) (end 42.774999 72.725001) (width 0.25) (layer F.Cu) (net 12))
 (segment (start 44 47.3) (end 42.774999 48.525001) (width 0.25) (layer F.Cu) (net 12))
 (segment (start 41.5 79.151472) (end 41.5 80) (width 0.25) (layer F.Cu) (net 12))
 (segment (start 41.5 74) (end 41.5 79.151472) (width 0.25) (layer F.Cu) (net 12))
 (segment (start 42.774999 72.725001) (end 41.5 74) (width 0.25) (layer F.Cu) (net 12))
 (segment (start 46.54 52.38) (end 46.54 54.04) (width 0.25) (layer B.Cu) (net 11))
 (segment (start 46.54 54.04) (end 60.5 68) (width 0.25) (layer B.Cu) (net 11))
 (segment (start 84.8 79.151472) (end 84.8 80) (width 0.25) (layer B.Cu) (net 11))
 (segment (start 84.8 78.46359) (end 84.8 79.151472) (width 0.25) (layer B.Cu) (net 11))
 (segment (start 74.33641 68) (end 84.8 78.46359) (width 0.25) (layer B.Cu) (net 11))
 (segment (start 60.5 68) (end 74.33641 68) (width 0.25) (layer B.Cu) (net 11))
 (segment (start 58.54 52.38) (end 71.56 65.4) (width 0.25) (layer B.Cu) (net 15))
 (segment (start 86.8 79.151472) (end 86.8 80) (width 0.25) (layer B.Cu) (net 15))
 (segment (start 86.8 77.96359) (end 86.8 79.151472) (width 0.25) (layer B.Cu) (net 15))
 (segment (start 74.23641 65.4) (end 86.8 77.96359) (width 0.25) (layer B.Cu) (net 15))
 (segment (start 71.56 65.4) (end 74.23641 65.4) (width 0.25) (layer B.Cu) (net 15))
 (segment (start 88.8 79.151472) (end 88.8 80) (width 0.25) (layer B.Cu) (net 19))
 (segment (start 88.8 76.00359) (end 88.8 79.151472) (width 0.25) (layer B.Cu) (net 19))
 (segment (start 75.225001 62.428591) (end 88.8 76.00359) (width 0.25) (layer B.Cu) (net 19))
 (segment (start 75.225001 57.065001) (end 75.225001 62.428591) (width 0.25) (layer B.Cu) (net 19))
 (segment (start 70.54 52.38) (end 75.225001 57.065001) (width 0.25) (layer B.Cu) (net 19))
 (segment (start 82.54 52.38) (end 82.54 66.24) (width 0.25) (layer B.Cu) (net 1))
 (segment (start 90.8 74.5) (end 90.8 80) (width 0.25) (layer B.Cu) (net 1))
 (segment (start 82.54 66.24) (end 90.8 74.5) (width 0.25) (layer B.Cu) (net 1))
 (segment (start 94.54 71.86) (end 94.54 52.38) (width 0.25) (layer B.Cu) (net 25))
 (segment (start 92.8 73.6) (end 94.54 71.86) (width 0.25) (layer B.Cu) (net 25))
 (segment (start 92.8 80) (end 92.8 73.6) (width 0.25) (layer B.Cu) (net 25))
 (segment (start 106.54 68.26) (end 94.8 80) (width 0.25) (layer B.Cu) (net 29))
 (segment (start 106.54 52.38) (end 106.54 68.26) (width 0.25) (layer B.Cu) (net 29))
 (segment (start 52.54 53.652792) (end 65.587208 66.7) (width 0.25) (layer B.Cu) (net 14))
 (segment (start 52.54 52.38) (end 52.54 53.652792) (width 0.25) (layer B.Cu) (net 14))
 (segment (start 65.587208 66.7) (end 74.9 66.7) (width 0.25) (layer B.Cu) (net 14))
 (segment (start 85.399999 81.400001) (end 84.8 82) (width 0.25) (layer B.Cu) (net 14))
 (segment (start 85.725001 81.074999) (end 85.399999 81.400001) (width 0.25) (layer B.Cu) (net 14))
 (segment (start 85.725001 77.525001) (end 85.725001 81.074999) (width 0.25) (layer B.Cu) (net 14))
 (segment (start 74.9 66.7) (end 85.725001 77.525001) (width 0.25) (layer B.Cu) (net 14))
 (segment (start 87.399999 81.400001) (end 86.8 82) (width 0.25) (layer B.Cu) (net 18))
 (segment (start 87.725001 81.074999) (end 87.399999 81.400001) (width 0.25) (layer B.Cu) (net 18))
 (segment (start 87.725001 75.565001) (end 87.725001 81.074999) (width 0.25) (layer B.Cu) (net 18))
 (segment (start 64.54 52.38) (end 87.725001 75.565001) (width 0.25) (layer B.Cu) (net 18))
 (segment (start 76.54 52.38) (end 76.54 61.84) (width 0.25) (layer B.Cu) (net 22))
 (segment (start 89.399999 81.400001) (end 88.8 82) (width 0.25) (layer B.Cu) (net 22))
 (segment (start 89.725001 81.074999) (end 89.399999 81.400001) (width 0.25) (layer B.Cu) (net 22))
 (segment (start 89.725001 75.025001) (end 89.725001 81.074999) (width 0.25) (layer B.Cu) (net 22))
 (segment (start 76.54 61.84) (end 89.725001 75.025001) (width 0.25) (layer B.Cu) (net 22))
 (segment (start 88.54 52.38) (end 88.54 70.74) (width 0.25) (layer B.Cu) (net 23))
 (segment (start 91.399999 81.400001) (end 90.8 82) (width 0.25) (layer B.Cu) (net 23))
 (segment (start 91.725001 81.074999) (end 91.399999 81.400001) (width 0.25) (layer B.Cu) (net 23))
 (segment (start 91.725001 73.925001) (end 91.725001 81.074999) (width 0.25) (layer B.Cu) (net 23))
 (segment (start 88.54 70.74) (end 91.725001 73.925001) (width 0.25) (layer B.Cu) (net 23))
 (segment (start 100.54 52.38) (end 100.54 67.56) (width 0.25) (layer B.Cu) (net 28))
 (segment (start 93.399999 81.400001) (end 92.8 82) (width 0.25) (layer B.Cu) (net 28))
 (segment (start 93.725001 81.074999) (end 93.399999 81.400001) (width 0.25) (layer B.Cu) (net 28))
 (segment (start 93.725001 74.374999) (end 93.725001 81.074999) (width 0.25) (layer B.Cu) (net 28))
 (segment (start 100.54 67.56) (end 93.725001 74.374999) (width 0.25) (layer B.Cu) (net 28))
 (segment (start 112.54 64.26) (end 94.8 82) (width 0.25) (layer B.Cu) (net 32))
 (segment (start 112.54 52.38) (end 112.54 64.26) (width 0.25) (layer B.Cu) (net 32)))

